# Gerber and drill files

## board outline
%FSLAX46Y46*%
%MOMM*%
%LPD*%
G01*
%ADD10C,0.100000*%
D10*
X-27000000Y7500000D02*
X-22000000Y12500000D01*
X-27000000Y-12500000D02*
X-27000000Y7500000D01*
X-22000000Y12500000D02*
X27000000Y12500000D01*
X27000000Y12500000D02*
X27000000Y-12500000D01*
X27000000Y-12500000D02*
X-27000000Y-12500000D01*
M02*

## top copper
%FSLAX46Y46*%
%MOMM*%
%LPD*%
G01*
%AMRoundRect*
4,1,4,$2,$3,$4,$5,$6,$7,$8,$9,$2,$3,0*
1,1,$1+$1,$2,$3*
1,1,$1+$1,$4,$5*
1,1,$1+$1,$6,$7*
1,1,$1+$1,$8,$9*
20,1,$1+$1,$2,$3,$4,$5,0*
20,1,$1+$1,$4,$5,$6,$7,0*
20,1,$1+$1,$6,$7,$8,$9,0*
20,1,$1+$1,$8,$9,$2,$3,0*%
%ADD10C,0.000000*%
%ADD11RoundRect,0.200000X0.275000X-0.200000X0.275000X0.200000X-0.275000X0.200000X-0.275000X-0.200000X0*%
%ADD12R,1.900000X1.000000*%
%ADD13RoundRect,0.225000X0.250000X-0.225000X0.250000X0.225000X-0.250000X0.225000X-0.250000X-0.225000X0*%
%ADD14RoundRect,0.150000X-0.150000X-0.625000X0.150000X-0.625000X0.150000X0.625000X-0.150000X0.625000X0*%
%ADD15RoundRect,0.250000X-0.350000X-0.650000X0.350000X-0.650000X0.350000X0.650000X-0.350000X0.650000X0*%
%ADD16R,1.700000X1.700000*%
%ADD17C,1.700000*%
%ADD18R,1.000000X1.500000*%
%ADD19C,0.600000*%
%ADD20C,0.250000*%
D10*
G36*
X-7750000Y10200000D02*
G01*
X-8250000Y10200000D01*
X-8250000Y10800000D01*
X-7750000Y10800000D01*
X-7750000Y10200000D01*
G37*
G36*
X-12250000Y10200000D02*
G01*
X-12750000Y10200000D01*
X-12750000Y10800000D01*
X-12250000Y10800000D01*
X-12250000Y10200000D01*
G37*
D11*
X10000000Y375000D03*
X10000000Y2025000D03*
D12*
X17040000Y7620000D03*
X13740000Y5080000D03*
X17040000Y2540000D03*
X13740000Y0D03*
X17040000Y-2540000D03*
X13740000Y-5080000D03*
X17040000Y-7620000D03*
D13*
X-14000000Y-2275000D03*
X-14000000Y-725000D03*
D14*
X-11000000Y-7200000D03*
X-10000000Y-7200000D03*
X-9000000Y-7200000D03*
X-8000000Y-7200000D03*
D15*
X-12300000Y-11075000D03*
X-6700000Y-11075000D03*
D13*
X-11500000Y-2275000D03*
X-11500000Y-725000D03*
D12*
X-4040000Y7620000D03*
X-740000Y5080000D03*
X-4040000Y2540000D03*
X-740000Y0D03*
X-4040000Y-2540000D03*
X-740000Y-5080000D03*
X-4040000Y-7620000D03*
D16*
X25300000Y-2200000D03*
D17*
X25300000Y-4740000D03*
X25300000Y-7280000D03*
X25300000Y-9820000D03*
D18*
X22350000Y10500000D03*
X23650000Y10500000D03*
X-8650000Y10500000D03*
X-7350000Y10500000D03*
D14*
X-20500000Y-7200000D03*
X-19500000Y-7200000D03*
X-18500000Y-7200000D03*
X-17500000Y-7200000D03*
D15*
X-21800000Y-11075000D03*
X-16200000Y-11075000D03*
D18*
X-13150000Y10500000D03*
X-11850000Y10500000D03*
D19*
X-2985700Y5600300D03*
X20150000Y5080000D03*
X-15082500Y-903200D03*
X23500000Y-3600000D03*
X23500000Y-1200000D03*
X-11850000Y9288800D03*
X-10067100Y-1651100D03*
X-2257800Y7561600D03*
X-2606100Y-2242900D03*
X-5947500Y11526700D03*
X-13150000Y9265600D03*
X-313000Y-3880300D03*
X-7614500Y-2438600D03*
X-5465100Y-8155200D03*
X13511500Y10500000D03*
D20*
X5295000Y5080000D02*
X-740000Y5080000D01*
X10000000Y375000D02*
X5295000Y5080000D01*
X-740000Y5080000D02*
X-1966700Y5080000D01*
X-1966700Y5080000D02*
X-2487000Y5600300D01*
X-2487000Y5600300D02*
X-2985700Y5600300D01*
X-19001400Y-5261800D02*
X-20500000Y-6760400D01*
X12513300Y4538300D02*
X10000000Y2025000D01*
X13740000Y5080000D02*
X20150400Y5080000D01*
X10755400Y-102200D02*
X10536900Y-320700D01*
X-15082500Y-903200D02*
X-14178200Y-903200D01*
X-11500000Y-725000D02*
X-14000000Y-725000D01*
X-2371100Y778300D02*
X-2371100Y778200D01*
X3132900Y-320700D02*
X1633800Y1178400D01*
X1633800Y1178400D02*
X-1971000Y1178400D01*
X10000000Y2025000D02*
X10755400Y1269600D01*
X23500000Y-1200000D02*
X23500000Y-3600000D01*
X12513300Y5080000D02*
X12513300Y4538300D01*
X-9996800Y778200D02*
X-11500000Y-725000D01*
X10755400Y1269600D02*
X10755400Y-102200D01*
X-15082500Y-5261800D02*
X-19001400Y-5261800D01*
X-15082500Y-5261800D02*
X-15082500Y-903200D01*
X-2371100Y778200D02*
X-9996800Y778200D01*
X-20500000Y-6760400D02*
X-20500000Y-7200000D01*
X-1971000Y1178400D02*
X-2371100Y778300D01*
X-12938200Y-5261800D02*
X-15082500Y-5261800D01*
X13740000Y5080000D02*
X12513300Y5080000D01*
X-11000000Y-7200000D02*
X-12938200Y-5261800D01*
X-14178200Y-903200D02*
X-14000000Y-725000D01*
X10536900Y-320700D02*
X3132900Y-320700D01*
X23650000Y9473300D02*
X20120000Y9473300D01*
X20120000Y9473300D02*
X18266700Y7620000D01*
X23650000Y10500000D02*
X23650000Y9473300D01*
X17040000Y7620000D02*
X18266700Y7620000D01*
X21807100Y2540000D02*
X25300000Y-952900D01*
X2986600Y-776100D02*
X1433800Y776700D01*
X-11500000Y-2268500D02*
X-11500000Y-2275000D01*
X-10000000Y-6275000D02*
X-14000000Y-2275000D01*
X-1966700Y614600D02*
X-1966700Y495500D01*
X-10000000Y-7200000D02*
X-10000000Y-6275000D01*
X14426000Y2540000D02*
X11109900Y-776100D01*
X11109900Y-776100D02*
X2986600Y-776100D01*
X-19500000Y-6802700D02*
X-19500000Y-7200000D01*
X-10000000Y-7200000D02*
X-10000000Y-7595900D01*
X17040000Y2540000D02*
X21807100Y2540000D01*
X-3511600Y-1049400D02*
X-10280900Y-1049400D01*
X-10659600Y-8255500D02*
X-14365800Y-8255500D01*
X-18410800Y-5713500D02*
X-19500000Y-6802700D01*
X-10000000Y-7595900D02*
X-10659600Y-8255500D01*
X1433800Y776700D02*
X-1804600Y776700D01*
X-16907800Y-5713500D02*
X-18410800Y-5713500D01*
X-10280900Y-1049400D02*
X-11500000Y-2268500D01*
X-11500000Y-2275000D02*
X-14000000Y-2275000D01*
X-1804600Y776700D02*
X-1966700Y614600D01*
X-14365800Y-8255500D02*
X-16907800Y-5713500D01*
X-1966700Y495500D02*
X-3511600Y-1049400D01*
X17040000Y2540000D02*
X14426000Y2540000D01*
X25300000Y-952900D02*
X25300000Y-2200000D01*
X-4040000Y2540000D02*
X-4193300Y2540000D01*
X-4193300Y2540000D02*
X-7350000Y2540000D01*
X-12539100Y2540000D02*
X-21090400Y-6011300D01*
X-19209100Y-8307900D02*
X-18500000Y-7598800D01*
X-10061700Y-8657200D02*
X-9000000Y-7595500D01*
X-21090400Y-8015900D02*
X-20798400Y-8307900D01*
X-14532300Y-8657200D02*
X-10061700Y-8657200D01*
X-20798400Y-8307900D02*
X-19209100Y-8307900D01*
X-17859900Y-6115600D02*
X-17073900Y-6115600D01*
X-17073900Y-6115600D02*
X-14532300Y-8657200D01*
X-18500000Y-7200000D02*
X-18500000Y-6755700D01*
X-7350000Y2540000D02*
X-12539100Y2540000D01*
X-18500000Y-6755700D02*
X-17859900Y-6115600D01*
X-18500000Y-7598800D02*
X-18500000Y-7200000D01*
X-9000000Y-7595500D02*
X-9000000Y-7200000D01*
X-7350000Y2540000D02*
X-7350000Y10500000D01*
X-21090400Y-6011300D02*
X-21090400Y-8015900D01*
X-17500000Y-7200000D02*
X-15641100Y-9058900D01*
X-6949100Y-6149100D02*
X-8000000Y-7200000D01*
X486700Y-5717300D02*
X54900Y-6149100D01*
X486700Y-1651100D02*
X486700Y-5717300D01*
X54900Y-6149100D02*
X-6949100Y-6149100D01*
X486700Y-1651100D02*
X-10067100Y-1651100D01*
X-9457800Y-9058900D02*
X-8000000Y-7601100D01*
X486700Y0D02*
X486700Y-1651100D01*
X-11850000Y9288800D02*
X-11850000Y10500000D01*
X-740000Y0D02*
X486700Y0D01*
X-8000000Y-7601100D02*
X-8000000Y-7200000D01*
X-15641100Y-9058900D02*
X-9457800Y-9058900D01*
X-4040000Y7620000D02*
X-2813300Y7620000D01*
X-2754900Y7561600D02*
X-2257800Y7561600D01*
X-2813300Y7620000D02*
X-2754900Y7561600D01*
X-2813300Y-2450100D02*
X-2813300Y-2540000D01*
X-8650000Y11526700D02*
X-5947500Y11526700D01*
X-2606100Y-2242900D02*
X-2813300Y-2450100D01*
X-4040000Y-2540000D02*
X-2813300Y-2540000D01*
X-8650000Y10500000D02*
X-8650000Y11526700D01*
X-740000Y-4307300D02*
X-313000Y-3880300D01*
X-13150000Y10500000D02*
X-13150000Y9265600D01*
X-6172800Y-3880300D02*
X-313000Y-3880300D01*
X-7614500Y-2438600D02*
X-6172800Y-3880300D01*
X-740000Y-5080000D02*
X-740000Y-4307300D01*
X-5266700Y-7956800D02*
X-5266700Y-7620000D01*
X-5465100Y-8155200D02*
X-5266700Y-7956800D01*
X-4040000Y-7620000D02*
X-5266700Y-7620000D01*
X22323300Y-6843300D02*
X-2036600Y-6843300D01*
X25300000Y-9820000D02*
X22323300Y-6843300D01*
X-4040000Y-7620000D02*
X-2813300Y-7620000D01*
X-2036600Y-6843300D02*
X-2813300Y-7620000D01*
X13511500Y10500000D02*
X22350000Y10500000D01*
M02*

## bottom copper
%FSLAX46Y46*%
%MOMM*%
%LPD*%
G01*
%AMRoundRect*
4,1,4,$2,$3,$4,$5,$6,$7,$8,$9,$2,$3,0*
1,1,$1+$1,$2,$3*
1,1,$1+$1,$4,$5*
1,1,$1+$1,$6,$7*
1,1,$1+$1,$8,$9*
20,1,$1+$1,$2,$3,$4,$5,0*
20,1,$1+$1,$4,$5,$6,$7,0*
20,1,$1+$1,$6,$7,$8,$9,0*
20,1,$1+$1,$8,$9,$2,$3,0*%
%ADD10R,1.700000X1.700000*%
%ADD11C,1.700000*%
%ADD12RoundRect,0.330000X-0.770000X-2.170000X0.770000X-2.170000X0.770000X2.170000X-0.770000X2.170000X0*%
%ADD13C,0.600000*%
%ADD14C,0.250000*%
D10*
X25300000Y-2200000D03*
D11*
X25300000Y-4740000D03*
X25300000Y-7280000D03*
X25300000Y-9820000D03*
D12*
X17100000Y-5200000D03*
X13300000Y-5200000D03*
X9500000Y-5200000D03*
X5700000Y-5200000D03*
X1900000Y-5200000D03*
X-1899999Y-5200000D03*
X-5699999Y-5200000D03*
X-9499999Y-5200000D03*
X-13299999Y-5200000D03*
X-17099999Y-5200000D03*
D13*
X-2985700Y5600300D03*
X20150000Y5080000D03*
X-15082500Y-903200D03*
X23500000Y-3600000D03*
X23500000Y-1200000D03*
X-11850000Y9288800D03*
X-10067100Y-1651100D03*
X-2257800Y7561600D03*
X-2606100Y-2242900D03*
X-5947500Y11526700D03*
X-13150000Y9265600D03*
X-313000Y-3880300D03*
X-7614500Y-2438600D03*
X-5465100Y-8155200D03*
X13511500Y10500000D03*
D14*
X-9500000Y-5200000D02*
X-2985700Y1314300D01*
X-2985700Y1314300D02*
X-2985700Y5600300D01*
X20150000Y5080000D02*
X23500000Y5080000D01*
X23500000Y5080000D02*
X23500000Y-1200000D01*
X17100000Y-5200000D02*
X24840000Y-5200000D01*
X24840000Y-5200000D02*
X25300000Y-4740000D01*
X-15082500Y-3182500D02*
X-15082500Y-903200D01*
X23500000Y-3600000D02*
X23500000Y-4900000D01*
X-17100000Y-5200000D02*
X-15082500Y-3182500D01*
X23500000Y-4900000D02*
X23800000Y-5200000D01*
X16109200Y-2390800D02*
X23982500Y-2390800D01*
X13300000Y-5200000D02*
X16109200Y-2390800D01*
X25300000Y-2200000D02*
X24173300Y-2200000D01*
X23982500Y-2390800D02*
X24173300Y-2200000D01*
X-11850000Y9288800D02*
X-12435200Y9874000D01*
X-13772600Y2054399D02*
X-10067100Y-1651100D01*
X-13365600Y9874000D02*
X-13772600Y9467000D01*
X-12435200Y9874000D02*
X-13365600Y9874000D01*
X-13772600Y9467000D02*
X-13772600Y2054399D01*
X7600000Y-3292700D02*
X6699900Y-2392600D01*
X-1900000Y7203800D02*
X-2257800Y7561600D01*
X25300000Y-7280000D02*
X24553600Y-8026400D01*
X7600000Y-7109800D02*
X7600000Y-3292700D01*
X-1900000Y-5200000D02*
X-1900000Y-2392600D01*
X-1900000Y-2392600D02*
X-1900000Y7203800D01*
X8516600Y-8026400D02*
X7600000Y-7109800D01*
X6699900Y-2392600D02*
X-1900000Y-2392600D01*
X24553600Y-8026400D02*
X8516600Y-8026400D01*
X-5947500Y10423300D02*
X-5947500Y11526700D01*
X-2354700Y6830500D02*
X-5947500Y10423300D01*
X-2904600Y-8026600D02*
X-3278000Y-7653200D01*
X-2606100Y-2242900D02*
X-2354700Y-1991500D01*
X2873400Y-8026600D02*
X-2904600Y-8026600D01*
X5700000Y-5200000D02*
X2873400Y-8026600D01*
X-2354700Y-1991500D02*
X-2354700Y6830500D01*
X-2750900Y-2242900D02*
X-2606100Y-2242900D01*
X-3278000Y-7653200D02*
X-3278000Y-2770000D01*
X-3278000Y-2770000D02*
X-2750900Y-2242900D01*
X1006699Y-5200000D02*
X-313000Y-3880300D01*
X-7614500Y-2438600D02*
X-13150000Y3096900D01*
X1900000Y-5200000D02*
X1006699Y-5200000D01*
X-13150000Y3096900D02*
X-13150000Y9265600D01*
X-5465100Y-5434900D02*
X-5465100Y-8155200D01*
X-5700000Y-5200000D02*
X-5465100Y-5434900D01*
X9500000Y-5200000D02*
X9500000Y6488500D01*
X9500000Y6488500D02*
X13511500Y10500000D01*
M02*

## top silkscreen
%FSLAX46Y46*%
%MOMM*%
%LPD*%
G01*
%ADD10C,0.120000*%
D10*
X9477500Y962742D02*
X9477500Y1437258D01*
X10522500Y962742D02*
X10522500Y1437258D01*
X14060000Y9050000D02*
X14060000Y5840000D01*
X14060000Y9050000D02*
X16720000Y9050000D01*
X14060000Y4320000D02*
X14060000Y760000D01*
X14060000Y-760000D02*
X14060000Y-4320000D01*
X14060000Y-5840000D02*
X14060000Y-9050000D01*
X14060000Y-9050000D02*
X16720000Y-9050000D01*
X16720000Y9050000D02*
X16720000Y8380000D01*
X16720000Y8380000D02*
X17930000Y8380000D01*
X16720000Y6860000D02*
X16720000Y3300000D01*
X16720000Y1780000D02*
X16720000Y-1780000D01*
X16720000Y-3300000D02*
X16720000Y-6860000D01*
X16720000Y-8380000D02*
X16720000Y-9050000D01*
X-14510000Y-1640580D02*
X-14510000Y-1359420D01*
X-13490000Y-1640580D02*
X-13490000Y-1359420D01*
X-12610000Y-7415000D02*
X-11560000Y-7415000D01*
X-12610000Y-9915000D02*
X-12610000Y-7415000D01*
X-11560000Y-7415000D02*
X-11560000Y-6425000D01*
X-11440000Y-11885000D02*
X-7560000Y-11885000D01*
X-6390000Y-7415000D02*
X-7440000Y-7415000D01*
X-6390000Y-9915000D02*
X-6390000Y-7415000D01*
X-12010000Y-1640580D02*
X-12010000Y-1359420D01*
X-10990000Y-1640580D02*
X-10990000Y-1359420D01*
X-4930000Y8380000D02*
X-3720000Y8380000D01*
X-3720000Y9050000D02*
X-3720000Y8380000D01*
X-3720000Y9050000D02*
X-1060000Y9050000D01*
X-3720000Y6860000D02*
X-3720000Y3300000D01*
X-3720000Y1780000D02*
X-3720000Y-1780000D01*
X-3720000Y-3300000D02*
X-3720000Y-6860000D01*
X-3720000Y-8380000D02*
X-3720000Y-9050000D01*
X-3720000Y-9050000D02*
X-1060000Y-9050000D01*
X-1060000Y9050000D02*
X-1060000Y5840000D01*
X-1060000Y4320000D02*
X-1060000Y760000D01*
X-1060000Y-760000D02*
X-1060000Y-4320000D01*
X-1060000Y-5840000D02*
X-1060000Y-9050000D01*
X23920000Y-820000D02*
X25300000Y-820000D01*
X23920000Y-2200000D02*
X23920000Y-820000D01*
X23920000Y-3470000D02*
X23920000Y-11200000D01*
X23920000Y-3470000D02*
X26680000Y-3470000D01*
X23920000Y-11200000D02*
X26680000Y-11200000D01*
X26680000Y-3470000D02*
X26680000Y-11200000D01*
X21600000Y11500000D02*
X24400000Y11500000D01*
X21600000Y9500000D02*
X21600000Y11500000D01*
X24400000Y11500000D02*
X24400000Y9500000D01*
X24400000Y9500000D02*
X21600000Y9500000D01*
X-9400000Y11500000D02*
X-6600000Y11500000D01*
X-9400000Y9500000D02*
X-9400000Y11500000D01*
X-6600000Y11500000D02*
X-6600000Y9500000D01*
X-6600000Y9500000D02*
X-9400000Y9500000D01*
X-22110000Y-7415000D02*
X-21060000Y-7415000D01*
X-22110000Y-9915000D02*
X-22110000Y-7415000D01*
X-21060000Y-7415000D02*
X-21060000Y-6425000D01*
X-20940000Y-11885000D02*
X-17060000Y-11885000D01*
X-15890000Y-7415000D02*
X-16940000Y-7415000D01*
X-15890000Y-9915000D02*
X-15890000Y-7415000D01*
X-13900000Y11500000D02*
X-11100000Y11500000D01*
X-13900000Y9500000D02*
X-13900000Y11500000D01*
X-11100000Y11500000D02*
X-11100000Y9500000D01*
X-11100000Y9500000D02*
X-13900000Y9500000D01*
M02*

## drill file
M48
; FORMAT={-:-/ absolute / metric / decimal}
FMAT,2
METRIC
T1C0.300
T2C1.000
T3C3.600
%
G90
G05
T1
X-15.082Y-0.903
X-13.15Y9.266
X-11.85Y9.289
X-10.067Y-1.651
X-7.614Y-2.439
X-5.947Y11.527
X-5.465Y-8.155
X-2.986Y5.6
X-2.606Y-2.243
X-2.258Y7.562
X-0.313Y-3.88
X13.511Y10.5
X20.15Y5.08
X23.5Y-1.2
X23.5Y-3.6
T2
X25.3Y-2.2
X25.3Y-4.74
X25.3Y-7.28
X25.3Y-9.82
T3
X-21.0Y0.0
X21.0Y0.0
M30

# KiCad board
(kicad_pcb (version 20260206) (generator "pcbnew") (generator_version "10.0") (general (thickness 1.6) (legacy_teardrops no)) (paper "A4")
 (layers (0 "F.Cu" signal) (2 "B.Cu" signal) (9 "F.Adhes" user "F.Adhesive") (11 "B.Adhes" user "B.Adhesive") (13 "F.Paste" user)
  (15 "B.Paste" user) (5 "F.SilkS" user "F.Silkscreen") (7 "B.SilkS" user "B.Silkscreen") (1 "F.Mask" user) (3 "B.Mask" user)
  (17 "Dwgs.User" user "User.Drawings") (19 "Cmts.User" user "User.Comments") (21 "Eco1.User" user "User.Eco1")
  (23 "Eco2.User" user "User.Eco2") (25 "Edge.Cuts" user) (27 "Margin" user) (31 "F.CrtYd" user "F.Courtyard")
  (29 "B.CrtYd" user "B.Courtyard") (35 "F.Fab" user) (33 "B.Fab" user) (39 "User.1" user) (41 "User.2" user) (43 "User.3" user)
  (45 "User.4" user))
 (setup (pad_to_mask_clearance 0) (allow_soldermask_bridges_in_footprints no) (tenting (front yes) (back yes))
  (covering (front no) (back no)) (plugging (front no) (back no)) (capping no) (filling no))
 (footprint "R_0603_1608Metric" (layer "F.Cu") (at 10 -1.2 90)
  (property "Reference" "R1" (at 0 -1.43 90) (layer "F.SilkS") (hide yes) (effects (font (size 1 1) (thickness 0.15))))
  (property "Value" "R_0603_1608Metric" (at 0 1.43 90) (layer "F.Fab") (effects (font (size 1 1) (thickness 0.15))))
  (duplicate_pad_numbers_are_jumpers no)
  (fp_line (start -0.237258 -0.5225) (end 0.237258 -0.5225) (stroke (width 0.12) (type solid)) (layer "F.SilkS"))
  (fp_line (start -0.237258 0.5225) (end 0.237258 0.5225) (stroke (width 0.12) (type solid)) (layer "F.SilkS"))
  (pad "1" smd roundrect (at -0.825 0 90) (size 0.8 0.95) (layers "F.Cu" "F.Mask" "F.Paste") (roundrect_rratio 0.25) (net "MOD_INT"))
  (pad "2" smd roundrect (at 0.825 0 90) (size 0.8 0.95) (layers "F.Cu" "F.Mask" "F.Paste") (roundrect_rratio 0.25) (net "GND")))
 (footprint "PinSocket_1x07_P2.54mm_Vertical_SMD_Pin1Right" (layer "F.Cu") (at 15.39 0)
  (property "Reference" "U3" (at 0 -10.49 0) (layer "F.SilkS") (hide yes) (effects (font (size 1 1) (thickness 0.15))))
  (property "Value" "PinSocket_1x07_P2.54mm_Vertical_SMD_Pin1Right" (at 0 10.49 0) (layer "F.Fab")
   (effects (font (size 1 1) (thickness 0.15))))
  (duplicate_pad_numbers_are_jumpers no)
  (fp_line (start -1.33 -9.05) (end -1.33 -5.84) (stroke (width 0.12) (type solid)) (layer "F.SilkS"))
  (fp_line (start -1.33 -9.05) (end 1.33 -9.05) (stroke (width 0.12) (type solid)) (layer "F.SilkS"))
  (fp_line (start -1.33 -4.32) (end -1.33 -0.76) (stroke (width 0.12) (type solid)) (layer "F.SilkS"))
  (fp_line (start -1.33 0.76) (end -1.33 4.32) (stroke (width 0.12) (type solid)) (layer "F.SilkS"))
  (fp_line (start -1.33 5.84) (end -1.33 9.05) (stroke (width 0.12) (type solid)) (layer "F.SilkS"))
  (fp_line (start -1.33 9.05) (end 1.33 9.05) (stroke (width 0.12) (type solid)) (layer "F.SilkS"))
  (fp_line (start 1.33 -9.05) (end 1.33 -8.38) (stroke (width 0.12) (type solid)) (layer "F.SilkS"))
  (fp_line (start 1.33 -8.38) (end 2.54 -8.38) (stroke (width 0.12) (type solid)) (layer "F.SilkS"))
  (fp_line (start 1.33 -6.86) (end 1.33 -3.3) (stroke (width 0.12) (type solid)) (layer "F.SilkS"))
  (fp_line (start 1.33 -1.78) (end 1.33 1.78) (stroke (width 0.12) (type solid)) (layer "F.SilkS"))
  (fp_line (start 1.33 3.3) (end 1.33 6.86) (stroke (width 0.12) (type solid)) (layer "F.SilkS"))
  (fp_line (start 1.33 8.38) (end 1.33 9.05) (stroke (width 0.12) (type solid)) (layer "F.SilkS"))
  (pad "1" smd rect (at 1.65 -7.62) (size 1.9 1) (layers "F.Cu" "F.Mask" "F.Paste") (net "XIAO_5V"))
  (pad "2" smd rect (at -1.65 -5.08) (size 1.9 1) (layers "F.Cu" "F.Mask" "F.Paste") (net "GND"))
  (pad "3" smd rect (at 1.65 -2.54) (size 1.9 1) (layers "F.Cu" "F.Mask" "F.Paste") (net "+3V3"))
  (pad "4" smd rect (at -1.65 0) (size 1.9 1) (layers "F.Cu" "F.Mask" "F.Paste"))
  (pad "5" smd rect (at 1.65 2.54) (size 1.9 1) (layers "F.Cu" "F.Mask" "F.Paste"))
  (pad "6" smd rect (at -1.65 5.08) (size 1.9 1) (layers "F.Cu" "F.Mask" "F.Paste"))
  (pad "7" smd rect (at 1.65 7.62) (size 1.9 1) (layers "F.Cu" "F.Mask" "F.Paste")))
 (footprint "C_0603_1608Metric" (layer "F.Cu") (at -14 1.5 90)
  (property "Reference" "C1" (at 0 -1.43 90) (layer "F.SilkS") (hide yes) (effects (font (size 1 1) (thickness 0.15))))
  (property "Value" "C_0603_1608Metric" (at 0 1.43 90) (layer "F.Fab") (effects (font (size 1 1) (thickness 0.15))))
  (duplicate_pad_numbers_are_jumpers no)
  (fp_line (start -0.14058 -0.51) (end 0.14058 -0.51) (stroke (width 0.12) (type solid)) (layer "F.SilkS"))
  (fp_line (start -0.14058 0.51) (end 0.14058 0.51) (stroke (width 0.12) (type solid)) (layer "F.SilkS"))
  (pad "1" smd roundrect (at -0.775 0 90) (size 0.9 0.95) (layers "F.Cu" "F.Mask" "F.Paste") (roundrect_rratio 0.25) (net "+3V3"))
  (pad "2" smd roundrect (at 0.775 0 90) (size 0.9 0.95) (layers "F.Cu" "F.Mask" "F.Paste") (roundrect_rratio 0.25) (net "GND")))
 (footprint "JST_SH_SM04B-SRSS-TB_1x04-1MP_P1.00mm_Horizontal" (layer "F.Cu") (at -9.5 9.2)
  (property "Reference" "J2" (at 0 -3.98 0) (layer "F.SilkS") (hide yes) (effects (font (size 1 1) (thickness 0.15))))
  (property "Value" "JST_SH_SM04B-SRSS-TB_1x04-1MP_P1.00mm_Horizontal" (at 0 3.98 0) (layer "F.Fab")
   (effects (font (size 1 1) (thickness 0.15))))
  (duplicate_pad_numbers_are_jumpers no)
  (fp_line (start -3.11 -1.785) (end -2.06 -1.785) (stroke (width 0.12) (type solid)) (layer "F.SilkS"))
  (fp_line (start -3.11 0.715) (end -3.11 -1.785) (stroke (width 0.12) (type solid)) (layer "F.SilkS"))
  (fp_line (start -2.06 -1.785) (end -2.06 -2.775) (stroke (width 0.12) (type solid)) (layer "F.SilkS"))
  (fp_line (start -1.94 2.685) (end 1.94 2.685) (stroke (width 0.12) (type solid)) (layer "F.SilkS"))
  (fp_line (start 3.11 -1.785) (end 2.06 -1.785) (stroke (width 0.12) (type solid)) (layer "F.SilkS"))
  (fp_line (start 3.11 0.715) (end 3.11 -1.785) (stroke (width 0.12) (type solid)) (layer "F.SilkS"))
  (pad "1" smd roundrect (at -1.5 -2) (size 0.6 1.55) (layers "F.Cu" "F.Mask" "F.Paste") (roundrect_rratio 0.25) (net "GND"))
  (pad "2" smd roundrect (at -0.5 -2) (size 0.6 1.55) (layers "F.Cu" "F.Mask" "F.Paste") (roundrect_rratio 0.25) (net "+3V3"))
  (pad "3" smd roundrect (at 0.5 -2) (size 0.6 1.55) (layers "F.Cu" "F.Mask" "F.Paste") (roundrect_rratio 0.25) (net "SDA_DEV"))
  (pad "4" smd roundrect (at 1.5 -2) (size 0.6 1.55) (layers "F.Cu" "F.Mask" "F.Paste") (roundrect_rratio 0.25) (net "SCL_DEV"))
  (pad "MP" smd roundrect (at -2.8 1.875) (size 1.2 1.8) (layers "F.Cu" "F.Mask" "F.Paste") (roundrect_rratio 0.208333))
  (pad "MP" smd roundrect (at 2.8 1.875) (size 1.2 1.8) (layers "F.Cu" "F.Mask" "F.Paste") (roundrect_rratio 0.208333)))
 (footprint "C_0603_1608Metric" (layer "F.Cu") (at -11.5 1.5 90)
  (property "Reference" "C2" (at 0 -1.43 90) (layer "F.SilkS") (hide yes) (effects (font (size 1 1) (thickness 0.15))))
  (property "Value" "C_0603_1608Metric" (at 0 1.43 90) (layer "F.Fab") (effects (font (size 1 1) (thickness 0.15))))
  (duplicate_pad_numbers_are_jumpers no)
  (fp_line (start -0.14058 -0.51) (end 0.14058 -0.51) (stroke (width 0.12) (type solid)) (layer "F.SilkS"))
  (fp_line (start -0.14058 0.51) (end 0.14058 0.51) (stroke (width 0.12) (type solid)) (layer "F.SilkS"))
  (pad "1" smd roundrect (at -0.775 0 90) (size 0.9 0.95) (layers "F.Cu" "F.Mask" "F.Paste") (roundrect_rratio 0.25) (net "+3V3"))
  (pad "2" smd roundrect (at 0.775 0 90) (size 0.9 0.95) (layers "F.Cu" "F.Mask" "F.Paste") (roundrect_rratio 0.25) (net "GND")))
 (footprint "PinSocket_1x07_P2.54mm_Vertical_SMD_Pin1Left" (layer "F.Cu") (at -2.39 0)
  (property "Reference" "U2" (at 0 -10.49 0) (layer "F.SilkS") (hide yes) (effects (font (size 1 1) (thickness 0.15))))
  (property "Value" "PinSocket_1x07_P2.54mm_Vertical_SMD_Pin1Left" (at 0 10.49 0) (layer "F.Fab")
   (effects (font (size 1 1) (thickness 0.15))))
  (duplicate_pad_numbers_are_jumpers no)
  (fp_line (start -2.54 -8.38) (end -1.33 -8.38) (stroke (width 0.12) (type solid)) (layer "F.SilkS"))
  (fp_line (start -1.33 -9.05) (end -1.33 -8.38) (stroke (width 0.12) (type solid)) (layer "F.SilkS"))
  (fp_line (start -1.33 -9.05) (end 1.33 -9.05) (stroke (width 0.12) (type solid)) (layer "F.SilkS"))
  (fp_line (start -1.33 -6.86) (end -1.33 -3.3) (stroke (width 0.12) (type solid)) (layer "F.SilkS"))
  (fp_line (start -1.33 -1.78) (end -1.33 1.78) (stroke (width 0.12) (type solid)) (layer "F.SilkS"))
  (fp_line (start -1.33 3.3) (end -1.33 6.86) (stroke (width 0.12) (type solid)) (layer "F.SilkS"))
  (fp_line (start -1.33 8.38) (end -1.33 9.05) (stroke (width 0.12) (type solid)) (layer "F.SilkS"))
  (fp_line (start -1.33 9.05) (end 1.33 9.05) (stroke (width 0.12) (type solid)) (layer "F.SilkS"))
  (fp_line (start 1.33 -9.05) (end 1.33 -5.84) (stroke (width 0.12) (type solid)) (layer "F.SilkS"))
  (fp_line (start 1.33 -4.32) (end 1.33 -0.76) (stroke (width 0.12) (type solid)) (layer "F.SilkS"))
  (fp_line (start 1.33 0.76) (end 1.33 4.32) (stroke (width 0.12) (type solid)) (layer "F.SilkS"))
  (fp_line (start 1.33 5.84) (end 1.33 9.05) (stroke (width 0.12) (type solid)) (layer "F.SilkS"))
  (pad "1" smd rect (at -1.65 -7.62) (size 1.9 1) (layers "F.Cu" "F.Mask" "F.Paste") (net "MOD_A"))
  (pad "2" smd rect (at 1.65 -5.08) (size 1.9 1) (layers "F.Cu" "F.Mask" "F.Paste") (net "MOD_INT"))
  (pad "3" smd rect (at -1.65 -2.54) (size 1.9 1) (layers "F.Cu" "F.Mask" "F.Paste") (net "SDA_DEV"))
  (pad "4" smd rect (at 1.65 0) (size 1.9 1) (layers "F.Cu" "F.Mask" "F.Paste") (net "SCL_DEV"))
  (pad "5" smd rect (at -1.65 2.54) (size 1.9 1) (layers "F.Cu" "F.Mask" "F.Paste") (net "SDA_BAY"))
  (pad "6" smd rect (at 1.65 5.08) (size 1.9 1) (layers "F.Cu" "F.Mask" "F.Paste") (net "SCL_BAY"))
  (pad "7" smd rect (at -1.65 7.62) (size 1.9 1) (layers "F.Cu" "F.Mask" "F.Paste") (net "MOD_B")))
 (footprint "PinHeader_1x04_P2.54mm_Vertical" (layer "F.Cu") (at 25.3 2.2)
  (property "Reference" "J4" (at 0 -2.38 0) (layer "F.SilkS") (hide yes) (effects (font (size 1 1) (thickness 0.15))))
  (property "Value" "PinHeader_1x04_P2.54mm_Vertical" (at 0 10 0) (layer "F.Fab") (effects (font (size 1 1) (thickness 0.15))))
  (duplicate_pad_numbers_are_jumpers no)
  (fp_line (start -1.38 -1.38) (end 0 -1.38) (stroke (width 0.12) (type solid)) (layer "F.SilkS"))
  (fp_line (start -1.38 0) (end -1.38 -1.38) (stroke (width 0.12) (type solid)) (layer "F.SilkS"))
  (fp_line (start -1.38 1.27) (end -1.38 9) (stroke (width 0.12) (type solid)) (layer "F.SilkS"))
  (fp_line (start -1.38 1.27) (end 1.38 1.27) (stroke (width 0.12) (type solid)) (layer "F.SilkS"))
  (fp_line (start -1.38 9) (end 1.38 9) (stroke (width 0.12) (type solid)) (layer "F.SilkS"))
  (fp_line (start 1.38 1.27) (end 1.38 9) (stroke (width 0.12) (type solid)) (layer "F.SilkS"))
  (pad "1" thru_hole rect (at 0 0) (size 1.7 1.7) (drill 1) (layers "*.Cu" "*.Mask") (remove_unused_layers no) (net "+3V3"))
  (pad "2" thru_hole circle (at 0 2.54) (size 1.7 1.7) (drill 1) (layers "*.Cu" "*.Mask") (remove_unused_layers no) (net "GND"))
  (pad "3" thru_hole circle (at 0 5.08) (size 1.7 1.7) (drill 1) (layers "*.Cu" "*.Mask") (remove_unused_layers no) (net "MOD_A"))
  (pad "4" thru_hole circle (at 0 7.62) (size 1.7 1.7) (drill 1) (layers "*.Cu" "*.Mask") (remove_unused_layers no) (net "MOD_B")))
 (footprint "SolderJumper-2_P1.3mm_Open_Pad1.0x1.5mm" (layer "F.Cu") (at 23 -10.5)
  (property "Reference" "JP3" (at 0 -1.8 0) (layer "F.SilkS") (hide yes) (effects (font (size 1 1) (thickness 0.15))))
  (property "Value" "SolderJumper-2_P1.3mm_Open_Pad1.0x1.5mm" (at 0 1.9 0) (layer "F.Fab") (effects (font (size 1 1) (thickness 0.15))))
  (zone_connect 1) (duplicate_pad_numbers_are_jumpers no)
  (fp_line (start -1.4 -1) (end 1.4 -1) (stroke (width 0.12) (type solid)) (layer "F.SilkS"))
  (fp_line (start -1.4 1) (end -1.4 -1) (stroke (width 0.12) (type solid)) (layer "F.SilkS"))
  (fp_line (start 1.4 -1) (end 1.4 1) (stroke (width 0.12) (type solid)) (layer "F.SilkS"))
  (fp_line (start 1.4 1) (end -1.4 1) (stroke (width 0.12) (type solid)) (layer "F.SilkS"))
  (pad "1" smd rect (at -0.65 0) (size 1 1.5) (layers "F.Cu" "F.Mask") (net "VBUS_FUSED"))
  (pad "2" smd rect (at 0.65 0) (size 1 1.5) (layers "F.Cu" "F.Mask") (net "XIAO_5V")))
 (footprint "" (layer "F.Cu") (at 0 0)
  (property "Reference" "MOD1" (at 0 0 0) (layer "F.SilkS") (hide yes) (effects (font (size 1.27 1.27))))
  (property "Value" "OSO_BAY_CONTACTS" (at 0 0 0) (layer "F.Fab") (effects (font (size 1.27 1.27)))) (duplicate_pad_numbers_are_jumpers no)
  (pad "" np_thru_hole circle (at -21 0) (size 3.6 3.6) (drill 3.6) (layers "*.Cu" "*.Mask"))
  (pad "" np_thru_hole circle (at 21 0) (size 3.6 3.6) (drill 3.6) (layers "*.Cu" "*.Mask"))
  (pad "1" smd roundrect (at 17.1 5.2) (size 2.2 5) (layers "B.Cu" "B.Mask") (roundrect_rratio 0.15) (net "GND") (thermal_bridge_angle 45))
  (pad "2" smd roundrect (at 13.3 5.2) (size 2.2 5) (layers "B.Cu" "B.Mask") (roundrect_rratio 0.15) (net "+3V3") (thermal_bridge_angle 45))
  (pad "3" smd roundrect (at 9.5 5.2) (size 2.2 5) (layers "B.Cu" "B.Mask") (roundrect_rratio 0.15) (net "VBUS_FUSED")
   (thermal_bridge_angle 45))
  (pad "4" smd roundrect (at 5.7 5.2) (size 2.2 5) (layers "B.Cu" "B.Mask") (roundrect_rratio 0.15) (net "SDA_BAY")
   (thermal_bridge_angle 45))
  (pad "5" smd roundrect (at 1.9 5.2) (size 2.2 5) (layers "B.Cu" "B.Mask") (roundrect_rratio 0.15) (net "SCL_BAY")
   (thermal_bridge_angle 45))
  (pad "6" smd roundrect (at -1.899999 5.2) (size 2.2 5) (layers "B.Cu" "B.Mask") (roundrect_rratio 0.15) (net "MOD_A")
   (thermal_bridge_angle 45))
  (pad "7" smd roundrect (at -5.699999 5.2) (size 2.2 5) (layers "B.Cu" "B.Mask") (roundrect_rratio 0.15) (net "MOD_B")
   (thermal_bridge_angle 45))
  (pad "8" smd roundrect (at -9.499999 5.2) (size 2.2 5) (layers "B.Cu" "B.Mask") (roundrect_rratio 0.15) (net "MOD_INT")
   (thermal_bridge_angle 45))
  (pad "9" smd roundrect (at -13.299999 5.2) (size 2.2 5) (layers "B.Cu" "B.Mask") (roundrect_rratio 0.15) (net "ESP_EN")
   (thermal_bridge_angle 45))
  (pad "10" smd roundrect (at -17.099999 5.2) (size 2.2 5) (layers "B.Cu" "B.Mask") (roundrect_rratio 0.15) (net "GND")
   (thermal_bridge_angle 45)))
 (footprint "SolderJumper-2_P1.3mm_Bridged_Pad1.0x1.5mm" (layer "F.Cu") (at -8 -10.5)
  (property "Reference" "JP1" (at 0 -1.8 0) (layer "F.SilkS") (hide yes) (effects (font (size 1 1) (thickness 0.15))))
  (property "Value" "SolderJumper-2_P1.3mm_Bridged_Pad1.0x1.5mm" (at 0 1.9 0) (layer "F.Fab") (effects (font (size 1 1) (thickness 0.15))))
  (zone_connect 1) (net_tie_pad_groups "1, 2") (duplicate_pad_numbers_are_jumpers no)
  (fp_poly (pts (xy -0.25 -0.3) (xy 0.25 -0.3) (xy 0.25 0.3) (xy -0.25 0.3)) (stroke (width 0) (type solid)) (fill yes) (layer "F.Cu"))
  (fp_line (start -1.4 -1) (end 1.4 -1) (stroke (width 0.12) (type solid)) (layer "F.SilkS"))
  (fp_line (start -1.4 1) (end -1.4 -1) (stroke (width 0.12) (type solid)) (layer "F.SilkS"))
  (fp_line (start 1.4 -1) (end 1.4 1) (stroke (width 0.12) (type solid)) (layer "F.SilkS"))
  (fp_line (start 1.4 1) (end -1.4 1) (stroke (width 0.12) (type solid)) (layer "F.SilkS"))
  (pad "1" smd rect (at -0.65 0) (size 1 1.5) (layers "F.Cu" "F.Mask") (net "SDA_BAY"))
  (pad "2" smd rect (at 0.65 0) (size 1 1.5) (layers "F.Cu" "F.Mask") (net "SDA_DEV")))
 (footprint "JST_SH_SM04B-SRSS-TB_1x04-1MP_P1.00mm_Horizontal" (layer "F.Cu") (at -19 9.2)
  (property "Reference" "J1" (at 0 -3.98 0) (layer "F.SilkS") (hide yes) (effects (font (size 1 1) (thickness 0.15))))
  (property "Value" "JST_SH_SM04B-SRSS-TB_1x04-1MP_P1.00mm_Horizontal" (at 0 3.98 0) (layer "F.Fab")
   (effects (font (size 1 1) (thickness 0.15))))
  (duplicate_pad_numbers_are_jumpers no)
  (fp_line (start -3.11 -1.785) (end -2.06 -1.785) (stroke (width 0.12) (type solid)) (layer "F.SilkS"))
  (fp_line (start -3.11 0.715) (end -3.11 -1.785) (stroke (width 0.12) (type solid)) (layer "F.SilkS"))
  (fp_line (start -2.06 -1.785) (end -2.06 -2.775) (stroke (width 0.12) (type solid)) (layer "F.SilkS"))
  (fp_line (start -1.94 2.685) (end 1.94 2.685) (stroke (width 0.12) (type solid)) (layer "F.SilkS"))
  (fp_line (start 3.11 -1.785) (end 2.06 -1.785) (stroke (width 0.12) (type solid)) (layer "F.SilkS"))
  (fp_line (start 3.11 0.715) (end 3.11 -1.785) (stroke (width 0.12) (type solid)) (layer "F.SilkS"))
  (pad "1" smd roundrect (at -1.5 -2) (size 0.6 1.55) (layers "F.Cu" "F.Mask" "F.Paste") (roundrect_rratio 0.25) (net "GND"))
  (pad "2" smd roundrect (at -0.5 -2) (size 0.6 1.55) (layers "F.Cu" "F.Mask" "F.Paste") (roundrect_rratio 0.25) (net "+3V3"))
  (pad "3" smd roundrect (at 0.5 -2) (size 0.6 1.55) (layers "F.Cu" "F.Mask" "F.Paste") (roundrect_rratio 0.25) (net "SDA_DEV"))
  (pad "4" smd roundrect (at 1.5 -2) (size 0.6 1.55) (layers "F.Cu" "F.Mask" "F.Paste") (roundrect_rratio 0.25) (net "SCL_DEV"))
  (pad "MP" smd roundrect (at -2.8 1.875) (size 1.2 1.8) (layers "F.Cu" "F.Mask" "F.Paste") (roundrect_rratio 0.208333))
  (pad "MP" smd roundrect (at 2.8 1.875) (size 1.2 1.8) (layers "F.Cu" "F.Mask" "F.Paste") (roundrect_rratio 0.208333)))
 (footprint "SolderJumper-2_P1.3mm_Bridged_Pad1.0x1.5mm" (layer "F.Cu") (at -12.5 -10.5)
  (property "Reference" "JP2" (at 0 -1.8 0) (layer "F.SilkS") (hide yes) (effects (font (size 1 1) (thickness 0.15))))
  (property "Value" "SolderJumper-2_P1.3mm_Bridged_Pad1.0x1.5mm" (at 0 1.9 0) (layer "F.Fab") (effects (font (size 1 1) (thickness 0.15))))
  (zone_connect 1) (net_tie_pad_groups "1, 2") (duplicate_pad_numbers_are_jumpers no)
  (fp_poly (pts (xy -0.25 -0.3) (xy 0.25 -0.3) (xy 0.25 0.3) (xy -0.25 0.3)) (stroke (width 0) (type solid)) (fill yes) (layer "F.Cu"))
  (fp_line (start -1.4 -1) (end 1.4 -1) (stroke (width 0.12) (type solid)) (layer "F.SilkS"))
  (fp_line (start -1.4 1) (end -1.4 -1) (stroke (width 0.12) (type solid)) (layer "F.SilkS"))
  (fp_line (start 1.4 -1) (end 1.4 1) (stroke (width 0.12) (type solid)) (layer "F.SilkS"))
  (fp_line (start 1.4 1) (end -1.4 1) (stroke (width 0.12) (type solid)) (layer "F.SilkS"))
  (pad "1" smd rect (at -0.65 0) (size 1 1.5) (layers "F.Cu" "F.Mask") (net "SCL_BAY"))
  (pad "2" smd rect (at 0.65 0) (size 1 1.5) (layers "F.Cu" "F.Mask") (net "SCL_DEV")))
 (gr_line (start -27 -7.5) (end -22 -12.5) (stroke (width 0.1) (type default)) (layer "Edge.Cuts"))
 (gr_line (start -27 12.5) (end -27 -7.5) (stroke (width 0.1) (type default)) (layer "Edge.Cuts"))
 (gr_line (start -22 -12.5) (end 27 -12.5) (stroke (width 0.1) (type default)) (layer "Edge.Cuts"))
 (gr_line (start 27 -12.5) (end 27 12.5) (stroke (width 0.1) (type default)) (layer "Edge.Cuts"))
 (gr_line (start 27 12.5) (end -27 12.5) (stroke (width 0.1) (type default)) (layer "Edge.Cuts"))
 (segment (start 5.295 -5.08) (end -0.74 -5.08) (width 0.25) (layer "F.Cu") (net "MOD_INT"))
 (segment (start 10 -0.375) (end 5.295 -5.08) (width 0.25) (layer "F.Cu") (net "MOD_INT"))
 (segment (start -0.74 -5.08) (end -1.9667 -5.08) (width 0.25) (layer "F.Cu") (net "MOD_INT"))
 (segment (start -1.9667 -5.08) (end -2.487 -5.6003) (width 0.25) (layer "F.Cu") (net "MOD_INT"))
 (segment (start -2.487 -5.6003) (end -2.9857 -5.6003) (width 0.25) (layer "F.Cu") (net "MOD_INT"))
 (via (at -2.9857 -5.6003) (size 0.6) (drill 0.3) (layers "F.Cu" "B.Cu") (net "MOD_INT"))
 (segment (start -9.5 5.2) (end -2.9857 -1.3143) (width 0.25) (layer "B.Cu") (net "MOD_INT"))
 (segment (start -2.9857 -1.3143) (end -2.9857 -5.6003) (width 0.25) (layer "B.Cu") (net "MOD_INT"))
 (segment (start -19.0014 5.2618) (end -20.5 6.7604) (width 0.25) (layer "F.Cu") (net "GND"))
 (segment (start 12.5133 -4.5383) (end 10 -2.025) (width 0.25) (layer "F.Cu") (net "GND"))
 (segment (start 13.74 -5.08) (end 20.1504 -5.08) (width 0.25) (layer "F.Cu") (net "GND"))
 (segment (start 10.7554 0.1022) (end 10.5369 0.3207) (width 0.25) (layer "F.Cu") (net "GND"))
 (segment (start -15.0825 0.9032) (end -14.1782 0.9032) (width 0.25) (layer "F.Cu") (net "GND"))
 (segment (start -11.5 0.725) (end -14 0.725) (width 0.25) (layer "F.Cu") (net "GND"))
 (segment (start -2.3711 -0.7783) (end -2.3711 -0.7782) (width 0.25) (layer "F.Cu") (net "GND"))
 (segment (start 3.1329 0.3207) (end 1.6338 -1.1784) (width 0.25) (layer "F.Cu") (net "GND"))
 (segment (start 1.6338 -1.1784) (end -1.971 -1.1784) (width 0.25) (layer "F.Cu") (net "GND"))
 (segment (start 10 -2.025) (end 10.7554 -1.2696) (width 0.25) (layer "F.Cu") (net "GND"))
 (segment (start 23.5 1.2) (end 23.5 3.6) (width 0.25) (layer "F.Cu") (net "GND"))
 (segment (start 12.5133 -5.08) (end 12.5133 -4.5383) (width 0.25) (layer "F.Cu") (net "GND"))
 (segment (start -9.9968 -0.7782) (end -11.5 0.725) (width 0.25) (layer "F.Cu") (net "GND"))
 (segment (start 10.7554 -1.2696) (end 10.7554 0.1022) (width 0.25) (layer "F.Cu") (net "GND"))
 (segment (start -15.0825 5.2618) (end -19.0014 5.2618) (width 0.25) (layer "F.Cu") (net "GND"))
 (segment (start -15.0825 5.2618) (end -15.0825 0.9032) (width 0.25) (layer "F.Cu") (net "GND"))
 (segment (start -2.3711 -0.7782) (end -9.9968 -0.7782) (width 0.25) (layer "F.Cu") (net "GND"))
 (segment (start -20.5 6.7604) (end -20.5 7.2) (width 0.25) (layer "F.Cu") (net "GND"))
 (segment (start -1.971 -1.1784) (end -2.3711 -0.7783) (width 0.25) (layer "F.Cu") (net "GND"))
 (segment (start -12.9382 5.2618) (end -15.0825 5.2618) (width 0.25) (layer "F.Cu") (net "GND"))
 (segment (start 13.74 -5.08) (end 12.5133 -5.08) (width 0.25) (layer "F.Cu") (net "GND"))
 (segment (start -11 7.2) (end -12.9382 5.2618) (width 0.25) (layer "F.Cu") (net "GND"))
 (segment (start -14.1782 0.9032) (end -14 0.725) (width 0.25) (layer "F.Cu") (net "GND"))
 (segment (start 10.5369 0.3207) (end 3.1329 0.3207) (width 0.25) (layer "F.Cu") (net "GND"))
 (via (at 20.15 -5.08) (size 0.6) (drill 0.3) (layers "F.Cu" "B.Cu") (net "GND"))
 (via (at -15.0825 0.9032) (size 0.6) (drill 0.3) (layers "F.Cu" "B.Cu") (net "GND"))
 (via (at 23.5 3.6) (size 0.6) (drill 0.3) (layers "F.Cu" "B.Cu") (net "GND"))
 (via (at 23.5 1.2) (size 0.6) (drill 0.3) (layers "F.Cu" "B.Cu") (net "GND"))
 (segment (start 20.15 -5.08) (end 23.5 -5.08) (width 0.25) (layer "B.Cu") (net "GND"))
 (segment (start 23.5 -5.08) (end 23.5 1.2) (width 0.25) (layer "B.Cu") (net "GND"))
 (segment (start 17.1 5.2) (end 24.84 5.2) (width 0.25) (layer "B.Cu") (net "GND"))
 (segment (start 24.84 5.2) (end 25.3 4.74) (width 0.25) (layer "B.Cu") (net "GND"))
 (segment (start -15.0825 3.1825) (end -15.0825 0.9032) (width 0.25) (layer "B.Cu") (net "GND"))
 (segment (start 23.5 3.6) (end 23.5 4.9) (width 0.25) (layer "B.Cu") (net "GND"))
 (segment (start -17.1 5.2) (end -15.0825 3.1825) (width 0.25) (layer "B.Cu") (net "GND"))
 (segment (start 23.5 4.9) (end 23.8 5.2) (width 0.25) (layer "B.Cu") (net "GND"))
 (segment (start 23.65 -9.4733) (end 20.12 -9.4733) (width 0.25) (layer "F.Cu") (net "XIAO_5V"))
 (segment (start 20.12 -9.4733) (end 18.2667 -7.62) (width 0.25) (layer "F.Cu") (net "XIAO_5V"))
 (segment (start 23.65 -10.5) (end 23.65 -9.4733) (width 0.25) (layer "F.Cu") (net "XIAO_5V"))
 (segment (start 17.04 -7.62) (end 18.2667 -7.62) (width 0.25) (layer "F.Cu") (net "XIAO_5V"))
 (segment (start 21.8071 -2.54) (end 25.3 0.9529) (width 0.25) (layer "F.Cu") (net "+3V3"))
 (segment (start 2.9866 0.7761) (end 1.4338 -0.7767) (width 0.25) (layer "F.Cu") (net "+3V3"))
 (segment (start -11.5 2.2685) (end -11.5 2.275) (width 0.25) (layer "F.Cu") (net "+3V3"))
 (segment (start -10 6.275) (end -14 2.275) (width 0.25) (layer "F.Cu") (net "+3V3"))
 (segment (start -1.9667 -0.6146) (end -1.9667 -0.4955) (width 0.25) (layer "F.Cu") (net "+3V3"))
 (segment (start -10 7.2) (end -10 6.275) (width 0.25) (layer "F.Cu") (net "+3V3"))
 (segment (start 14.426 -2.54) (end 11.1099 0.7761) (width 0.25) (layer "F.Cu") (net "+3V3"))
 (segment (start 11.1099 0.7761) (end 2.9866 0.7761) (width 0.25) (layer "F.Cu") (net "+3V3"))
 (segment (start -19.5 6.8027) (end -19.5 7.2) (width 0.25) (layer "F.Cu") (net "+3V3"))
 (segment (start -10 7.2) (end -10 7.5959) (width 0.25) (layer "F.Cu") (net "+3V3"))
 (segment (start 17.04 -2.54) (end 21.8071 -2.54) (width 0.25) (layer "F.Cu") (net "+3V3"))
 (segment (start -3.5116 1.0494) (end -10.2809 1.0494) (width 0.25) (layer "F.Cu") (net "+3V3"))
 (segment (start -10.6596 8.2555) (end -14.3658 8.2555) (width 0.25) (layer "F.Cu") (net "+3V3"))
 (segment (start -18.4108 5.7135) (end -19.5 6.8027) (width 0.25) (layer "F.Cu") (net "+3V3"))
 (segment (start -10 7.5959) (end -10.6596 8.2555) (width 0.25) (layer "F.Cu") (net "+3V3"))
 (segment (start 1.4338 -0.7767) (end -1.8046 -0.7767) (width 0.25) (layer "F.Cu") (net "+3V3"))
 (segment (start -16.9078 5.7135) (end -18.4108 5.7135) (width 0.25) (layer "F.Cu") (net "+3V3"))
 (segment (start -10.2809 1.0494) (end -11.5 2.2685) (width 0.25) (layer "F.Cu") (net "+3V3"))
 (segment (start -11.5 2.275) (end -14 2.275) (width 0.25) (layer "F.Cu") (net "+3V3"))
 (segment (start -1.8046 -0.7767) (end -1.9667 -0.6146) (width 0.25) (layer "F.Cu") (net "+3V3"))
 (segment (start -14.3658 8.2555) (end -16.9078 5.7135) (width 0.25) (layer "F.Cu") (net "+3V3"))
 (segment (start -1.9667 -0.4955) (end -3.5116 1.0494) (width 0.25) (layer "F.Cu") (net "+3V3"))
 (segment (start 17.04 -2.54) (end 14.426 -2.54) (width 0.25) (layer "F.Cu") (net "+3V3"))
 (segment (start 25.3 0.9529) (end 25.3 2.2) (width 0.25) (layer "F.Cu") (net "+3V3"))
 (segment (start 16.1092 2.3908) (end 23.9825 2.3908) (width 0.25) (layer "B.Cu") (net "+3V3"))
 (segment (start 13.3 5.2) (end 16.1092 2.3908) (width 0.25) (layer "B.Cu") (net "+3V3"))
 (segment (start 25.3 2.2) (end 24.1733 2.2) (width 0.25) (layer "B.Cu") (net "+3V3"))
 (segment (start 23.9825 2.3908) (end 24.1733 2.2) (width 0.25) (layer "B.Cu") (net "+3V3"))
 (segment (start -4.04 -2.54) (end -4.1933 -2.54) (width 0.25) (layer "F.Cu") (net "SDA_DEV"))
 (segment (start -4.1933 -2.54) (end -7.35 -2.54) (width 0.25) (layer "F.Cu") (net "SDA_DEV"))
 (segment (start -12.5391 -2.54) (end -21.0904 6.0113) (width 0.25) (layer "F.Cu") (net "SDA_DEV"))
 (segment (start -19.2091 8.3079) (end -18.5 7.5988) (width 0.25) (layer "F.Cu") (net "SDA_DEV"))
 (segment (start -10.0617 8.6572) (end -9 7.5955) (width 0.25) (layer "F.Cu") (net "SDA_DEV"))
 (segment (start -21.0904 8.0159) (end -20.7984 8.3079) (width 0.25) (layer "F.Cu") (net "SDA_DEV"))
 (segment (start -14.5323 8.6572) (end -10.0617 8.6572) (width 0.25) (layer "F.Cu") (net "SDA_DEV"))
 (segment (start -20.7984 8.3079) (end -19.2091 8.3079) (width 0.25) (layer "F.Cu") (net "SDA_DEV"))
 (segment (start -17.8599 6.1156) (end -17.0739 6.1156) (width 0.25) (layer "F.Cu") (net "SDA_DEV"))
 (segment (start -17.0739 6.1156) (end -14.5323 8.6572) (width 0.25) (layer "F.Cu") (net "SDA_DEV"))
 (segment (start -18.5 7.2) (end -18.5 6.7557) (width 0.25) (layer "F.Cu") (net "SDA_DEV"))
 (segment (start -7.35 -2.54) (end -12.5391 -2.54) (width 0.25) (layer "F.Cu") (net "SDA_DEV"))
 (segment (start -18.5 6.7557) (end -17.8599 6.1156) (width 0.25) (layer "F.Cu") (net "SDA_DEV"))
 (segment (start -18.5 7.5988) (end -18.5 7.2) (width 0.25) (layer "F.Cu") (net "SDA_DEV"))
 (segment (start -9 7.5955) (end -9 7.2) (width 0.25) (layer "F.Cu") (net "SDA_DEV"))
 (segment (start -7.35 -2.54) (end -7.35 -10.5) (width 0.25) (layer "F.Cu") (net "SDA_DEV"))
 (segment (start -21.0904 6.0113) (end -21.0904 8.0159) (width 0.25) (layer "F.Cu") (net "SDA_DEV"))
 (segment (start -17.5 7.2) (end -15.6411 9.0589) (width 0.25) (layer "F.Cu") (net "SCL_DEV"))
 (segment (start -6.9491 6.1491) (end -8 7.2) (width 0.25) (layer "F.Cu") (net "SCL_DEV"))
 (segment (start 0.4867 5.7173) (end 0.0549 6.1491) (width 0.25) (layer "F.Cu") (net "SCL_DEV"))
 (segment (start 0.4867 1.6511) (end 0.4867 5.7173) (width 0.25) (layer "F.Cu") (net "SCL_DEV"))
 (segment (start 0.0549 6.1491) (end -6.9491 6.1491) (width 0.25) (layer "F.Cu") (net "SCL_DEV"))
 (segment (start 0.4867 1.6511) (end -10.0671 1.6511) (width 0.25) (layer "F.Cu") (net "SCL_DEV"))
 (segment (start -9.4578 9.0589) (end -8 7.6011) (width 0.25) (layer "F.Cu") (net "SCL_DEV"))
 (segment (start 0.4867 0) (end 0.4867 1.6511) (width 0.25) (layer "F.Cu") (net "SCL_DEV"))
 (segment (start -11.85 -9.2888) (end -11.85 -10.5) (width 0.25) (layer "F.Cu") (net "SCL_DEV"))
 (segment (start -0.74 0) (end 0.4867 0) (width 0.25) (layer "F.Cu") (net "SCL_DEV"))
 (segment (start -8 7.6011) (end -8 7.2) (width 0.25) (layer "F.Cu") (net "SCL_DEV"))
 (segment (start -15.6411 9.0589) (end -9.4578 9.0589) (width 0.25) (layer "F.Cu") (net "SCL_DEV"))
 (via (at -11.85 -9.2888) (size 0.6) (drill 0.3) (layers "F.Cu" "B.Cu") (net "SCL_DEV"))
 (via (at -10.0671 1.6511) (size 0.6) (drill 0.3) (layers "F.Cu" "B.Cu") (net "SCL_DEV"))
 (segment (start -11.85 -9.2888) (end -12.4352 -9.874) (width 0.25) (layer "B.Cu") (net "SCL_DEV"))
 (segment (start -13.7726 -2.054399) (end -10.0671 1.6511) (width 0.25) (layer "B.Cu") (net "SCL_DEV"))
 (segment (start -13.3656 -9.874) (end -13.7726 -9.467) (width 0.25) (layer "B.Cu") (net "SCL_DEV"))
 (segment (start -12.4352 -9.874) (end -13.3656 -9.874) (width 0.25) (layer "B.Cu") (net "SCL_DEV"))
 (segment (start -13.7726 -9.467) (end -13.7726 -2.054399) (width 0.25) (layer "B.Cu") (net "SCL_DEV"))
 (segment (start -4.04 -7.62) (end -2.8133 -7.62) (width 0.25) (layer "F.Cu") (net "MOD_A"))
 (segment (start -2.7549 -7.5616) (end -2.2578 -7.5616) (width 0.25) (layer "F.Cu") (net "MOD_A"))
 (segment (start -2.8133 -7.62) (end -2.7549 -7.5616) (width 0.25) (layer "F.Cu") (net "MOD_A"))
 (via (at -2.2578 -7.5616) (size 0.6) (drill 0.3) (layers "F.Cu" "B.Cu") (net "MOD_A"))
 (segment (start 7.6 3.2927) (end 6.6999 2.3926) (width 0.25) (layer "B.Cu") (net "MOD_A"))
 (segment (start -1.9 -7.2038) (end -2.2578 -7.5616) (width 0.25) (layer "B.Cu") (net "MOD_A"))
 (segment (start 25.3 7.28) (end 24.5536 8.0264) (width 0.25) (layer "B.Cu") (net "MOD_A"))
 (segment (start 7.6 7.1098) (end 7.6 3.2927) (width 0.25) (layer "B.Cu") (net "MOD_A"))
 (segment (start -1.9 5.2) (end -1.9 2.3926) (width 0.25) (layer "B.Cu") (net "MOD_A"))
 (segment (start -1.9 2.3926) (end -1.9 -7.2038) (width 0.25) (layer "B.Cu") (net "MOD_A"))
 (segment (start 8.5166 8.0264) (end 7.6 7.1098) (width 0.25) (layer "B.Cu") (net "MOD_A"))
 (segment (start 6.6999 2.3926) (end -1.9 2.3926) (width 0.25) (layer "B.Cu") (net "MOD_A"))
 (segment (start 24.5536 8.0264) (end 8.5166 8.0264) (width 0.25) (layer "B.Cu") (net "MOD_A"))
 (segment (start -2.8133 2.4501) (end -2.8133 2.54) (width 0.25) (layer "F.Cu") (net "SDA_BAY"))
 (segment (start -8.65 -11.5267) (end -5.9475 -11.5267) (width 0.25) (layer "F.Cu") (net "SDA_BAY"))
 (segment (start -2.6061 2.2429) (end -2.8133 2.4501) (width 0.25) (layer "F.Cu") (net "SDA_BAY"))
 (segment (start -4.04 2.54) (end -2.8133 2.54) (width 0.25) (layer "F.Cu") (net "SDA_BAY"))
 (segment (start -8.65 -10.5) (end -8.65 -11.5267) (width 0.25) (layer "F.Cu") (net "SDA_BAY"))
 (via (at -2.6061 2.2429) (size 0.6) (drill 0.3) (layers "F.Cu" "B.Cu") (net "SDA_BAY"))
 (via (at -5.9475 -11.5267) (size 0.6) (drill 0.3) (layers "F.Cu" "B.Cu") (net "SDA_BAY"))
 (segment (start -5.9475 -10.4233) (end -5.9475 -11.5267) (width 0.25) (layer "B.Cu") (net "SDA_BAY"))
 (segment (start -2.3547 -6.8305) (end -5.9475 -10.4233) (width 0.25) (layer "B.Cu") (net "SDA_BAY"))
 (segment (start -2.9046 8.0266) (end -3.278 7.6532) (width 0.25) (layer "B.Cu") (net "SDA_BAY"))
 (segment (start -2.6061 2.2429) (end -2.3547 1.9915) (width 0.25) (layer "B.Cu") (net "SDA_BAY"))
 (segment (start 2.8734 8.0266) (end -2.9046 8.0266) (width 0.25) (layer "B.Cu") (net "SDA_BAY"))
 (segment (start 5.7 5.2) (end 2.8734 8.0266) (width 0.25) (layer "B.Cu") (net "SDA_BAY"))
 (segment (start -2.3547 1.9915) (end -2.3547 -6.8305) (width 0.25) (layer "B.Cu") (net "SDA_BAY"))
 (segment (start -2.7509 2.2429) (end -2.6061 2.2429) (width 0.25) (layer "B.Cu") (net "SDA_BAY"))
 (segment (start -3.278 7.6532) (end -3.278 2.77) (width 0.25) (layer "B.Cu") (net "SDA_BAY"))
 (segment (start -3.278 2.77) (end -2.7509 2.2429) (width 0.25) (layer "B.Cu") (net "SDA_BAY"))
 (segment (start -0.74 4.3073) (end -0.313 3.8803) (width 0.25) (layer "F.Cu") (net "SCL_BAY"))
 (segment (start -13.15 -10.5) (end -13.15 -9.2656) (width 0.25) (layer "F.Cu") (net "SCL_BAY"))
 (segment (start -6.1728 3.8803) (end -0.313 3.8803) (width 0.25) (layer "F.Cu") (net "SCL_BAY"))
 (segment (start -7.6145 2.4386) (end -6.1728 3.8803) (width 0.25) (layer "F.Cu") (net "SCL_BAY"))
 (segment (start -0.74 5.08) (end -0.74 4.3073) (width 0.25) (layer "F.Cu") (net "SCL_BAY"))
 (via (at -13.15 -9.2656) (size 0.6) (drill 0.3) (layers "F.Cu" "B.Cu") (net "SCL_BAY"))
 (via (at -0.313 3.8803) (size 0.6) (drill 0.3) (layers "F.Cu" "B.Cu") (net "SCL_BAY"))
 (via (at -7.6145 2.4386) (size 0.6) (drill 0.3) (layers "F.Cu" "B.Cu") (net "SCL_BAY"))
 (segment (start 1.006699 5.2) (end -0.313 3.8803) (width 0.25) (layer "B.Cu") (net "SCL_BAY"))
 (segment (start -7.6145 2.4386) (end -13.15 -3.0969) (width 0.25) (layer "B.Cu") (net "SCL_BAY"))
 (segment (start 1.9 5.2) (end 1.006699 5.2) (width 0.25) (layer "B.Cu") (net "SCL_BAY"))
 (segment (start -13.15 -3.0969) (end -13.15 -9.2656) (width 0.25) (layer "B.Cu") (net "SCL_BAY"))
 (segment (start -5.2667 7.9568) (end -5.2667 7.62) (width 0.25) (layer "F.Cu") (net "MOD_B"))
 (segment (start -5.4651 8.1552) (end -5.2667 7.9568) (width 0.25) (layer "F.Cu") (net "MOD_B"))
 (segment (start -4.04 7.62) (end -5.2667 7.62) (width 0.25) (layer "F.Cu") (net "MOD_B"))
 (segment (start 22.3233 6.8433) (end -2.0366 6.8433) (width 0.25) (layer "F.Cu") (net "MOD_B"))
 (segment (start 25.3 9.82) (end 22.3233 6.8433) (width 0.25) (layer "F.Cu") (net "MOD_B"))
 (segment (start -4.04 7.62) (end -2.8133 7.62) (width 0.25) (layer "F.Cu") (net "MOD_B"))
 (segment (start -2.0366 6.8433) (end -2.8133 7.62) (width 0.25) (layer "F.Cu") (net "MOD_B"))
 (via (at -5.4651 8.1552) (size 0.6) (drill 0.3) (layers "F.Cu" "B.Cu") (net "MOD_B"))
 (segment (start -5.4651 5.4349) (end -5.4651 8.1552) (width 0.25) (layer "B.Cu") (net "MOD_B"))
 (segment (start -5.7 5.2) (end -5.4651 5.4349) (width 0.25) (layer "B.Cu") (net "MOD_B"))
 (segment (start 13.5115 -10.5) (end 22.35 -10.5) (width 0.25) (layer "F.Cu") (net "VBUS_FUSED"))
 (via (at 13.5115 -10.5) (size 0.6) (drill 0.3) (layers "F.Cu" "B.Cu") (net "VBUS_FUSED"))
 (segment (start 9.5 5.2) (end 9.5 -6.4885) (width 0.25) (layer "B.Cu") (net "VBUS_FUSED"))
 (segment (start 9.5 -6.4885) (end 13.5115 -10.5) (width 0.25) (layer "B.Cu") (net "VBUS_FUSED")))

